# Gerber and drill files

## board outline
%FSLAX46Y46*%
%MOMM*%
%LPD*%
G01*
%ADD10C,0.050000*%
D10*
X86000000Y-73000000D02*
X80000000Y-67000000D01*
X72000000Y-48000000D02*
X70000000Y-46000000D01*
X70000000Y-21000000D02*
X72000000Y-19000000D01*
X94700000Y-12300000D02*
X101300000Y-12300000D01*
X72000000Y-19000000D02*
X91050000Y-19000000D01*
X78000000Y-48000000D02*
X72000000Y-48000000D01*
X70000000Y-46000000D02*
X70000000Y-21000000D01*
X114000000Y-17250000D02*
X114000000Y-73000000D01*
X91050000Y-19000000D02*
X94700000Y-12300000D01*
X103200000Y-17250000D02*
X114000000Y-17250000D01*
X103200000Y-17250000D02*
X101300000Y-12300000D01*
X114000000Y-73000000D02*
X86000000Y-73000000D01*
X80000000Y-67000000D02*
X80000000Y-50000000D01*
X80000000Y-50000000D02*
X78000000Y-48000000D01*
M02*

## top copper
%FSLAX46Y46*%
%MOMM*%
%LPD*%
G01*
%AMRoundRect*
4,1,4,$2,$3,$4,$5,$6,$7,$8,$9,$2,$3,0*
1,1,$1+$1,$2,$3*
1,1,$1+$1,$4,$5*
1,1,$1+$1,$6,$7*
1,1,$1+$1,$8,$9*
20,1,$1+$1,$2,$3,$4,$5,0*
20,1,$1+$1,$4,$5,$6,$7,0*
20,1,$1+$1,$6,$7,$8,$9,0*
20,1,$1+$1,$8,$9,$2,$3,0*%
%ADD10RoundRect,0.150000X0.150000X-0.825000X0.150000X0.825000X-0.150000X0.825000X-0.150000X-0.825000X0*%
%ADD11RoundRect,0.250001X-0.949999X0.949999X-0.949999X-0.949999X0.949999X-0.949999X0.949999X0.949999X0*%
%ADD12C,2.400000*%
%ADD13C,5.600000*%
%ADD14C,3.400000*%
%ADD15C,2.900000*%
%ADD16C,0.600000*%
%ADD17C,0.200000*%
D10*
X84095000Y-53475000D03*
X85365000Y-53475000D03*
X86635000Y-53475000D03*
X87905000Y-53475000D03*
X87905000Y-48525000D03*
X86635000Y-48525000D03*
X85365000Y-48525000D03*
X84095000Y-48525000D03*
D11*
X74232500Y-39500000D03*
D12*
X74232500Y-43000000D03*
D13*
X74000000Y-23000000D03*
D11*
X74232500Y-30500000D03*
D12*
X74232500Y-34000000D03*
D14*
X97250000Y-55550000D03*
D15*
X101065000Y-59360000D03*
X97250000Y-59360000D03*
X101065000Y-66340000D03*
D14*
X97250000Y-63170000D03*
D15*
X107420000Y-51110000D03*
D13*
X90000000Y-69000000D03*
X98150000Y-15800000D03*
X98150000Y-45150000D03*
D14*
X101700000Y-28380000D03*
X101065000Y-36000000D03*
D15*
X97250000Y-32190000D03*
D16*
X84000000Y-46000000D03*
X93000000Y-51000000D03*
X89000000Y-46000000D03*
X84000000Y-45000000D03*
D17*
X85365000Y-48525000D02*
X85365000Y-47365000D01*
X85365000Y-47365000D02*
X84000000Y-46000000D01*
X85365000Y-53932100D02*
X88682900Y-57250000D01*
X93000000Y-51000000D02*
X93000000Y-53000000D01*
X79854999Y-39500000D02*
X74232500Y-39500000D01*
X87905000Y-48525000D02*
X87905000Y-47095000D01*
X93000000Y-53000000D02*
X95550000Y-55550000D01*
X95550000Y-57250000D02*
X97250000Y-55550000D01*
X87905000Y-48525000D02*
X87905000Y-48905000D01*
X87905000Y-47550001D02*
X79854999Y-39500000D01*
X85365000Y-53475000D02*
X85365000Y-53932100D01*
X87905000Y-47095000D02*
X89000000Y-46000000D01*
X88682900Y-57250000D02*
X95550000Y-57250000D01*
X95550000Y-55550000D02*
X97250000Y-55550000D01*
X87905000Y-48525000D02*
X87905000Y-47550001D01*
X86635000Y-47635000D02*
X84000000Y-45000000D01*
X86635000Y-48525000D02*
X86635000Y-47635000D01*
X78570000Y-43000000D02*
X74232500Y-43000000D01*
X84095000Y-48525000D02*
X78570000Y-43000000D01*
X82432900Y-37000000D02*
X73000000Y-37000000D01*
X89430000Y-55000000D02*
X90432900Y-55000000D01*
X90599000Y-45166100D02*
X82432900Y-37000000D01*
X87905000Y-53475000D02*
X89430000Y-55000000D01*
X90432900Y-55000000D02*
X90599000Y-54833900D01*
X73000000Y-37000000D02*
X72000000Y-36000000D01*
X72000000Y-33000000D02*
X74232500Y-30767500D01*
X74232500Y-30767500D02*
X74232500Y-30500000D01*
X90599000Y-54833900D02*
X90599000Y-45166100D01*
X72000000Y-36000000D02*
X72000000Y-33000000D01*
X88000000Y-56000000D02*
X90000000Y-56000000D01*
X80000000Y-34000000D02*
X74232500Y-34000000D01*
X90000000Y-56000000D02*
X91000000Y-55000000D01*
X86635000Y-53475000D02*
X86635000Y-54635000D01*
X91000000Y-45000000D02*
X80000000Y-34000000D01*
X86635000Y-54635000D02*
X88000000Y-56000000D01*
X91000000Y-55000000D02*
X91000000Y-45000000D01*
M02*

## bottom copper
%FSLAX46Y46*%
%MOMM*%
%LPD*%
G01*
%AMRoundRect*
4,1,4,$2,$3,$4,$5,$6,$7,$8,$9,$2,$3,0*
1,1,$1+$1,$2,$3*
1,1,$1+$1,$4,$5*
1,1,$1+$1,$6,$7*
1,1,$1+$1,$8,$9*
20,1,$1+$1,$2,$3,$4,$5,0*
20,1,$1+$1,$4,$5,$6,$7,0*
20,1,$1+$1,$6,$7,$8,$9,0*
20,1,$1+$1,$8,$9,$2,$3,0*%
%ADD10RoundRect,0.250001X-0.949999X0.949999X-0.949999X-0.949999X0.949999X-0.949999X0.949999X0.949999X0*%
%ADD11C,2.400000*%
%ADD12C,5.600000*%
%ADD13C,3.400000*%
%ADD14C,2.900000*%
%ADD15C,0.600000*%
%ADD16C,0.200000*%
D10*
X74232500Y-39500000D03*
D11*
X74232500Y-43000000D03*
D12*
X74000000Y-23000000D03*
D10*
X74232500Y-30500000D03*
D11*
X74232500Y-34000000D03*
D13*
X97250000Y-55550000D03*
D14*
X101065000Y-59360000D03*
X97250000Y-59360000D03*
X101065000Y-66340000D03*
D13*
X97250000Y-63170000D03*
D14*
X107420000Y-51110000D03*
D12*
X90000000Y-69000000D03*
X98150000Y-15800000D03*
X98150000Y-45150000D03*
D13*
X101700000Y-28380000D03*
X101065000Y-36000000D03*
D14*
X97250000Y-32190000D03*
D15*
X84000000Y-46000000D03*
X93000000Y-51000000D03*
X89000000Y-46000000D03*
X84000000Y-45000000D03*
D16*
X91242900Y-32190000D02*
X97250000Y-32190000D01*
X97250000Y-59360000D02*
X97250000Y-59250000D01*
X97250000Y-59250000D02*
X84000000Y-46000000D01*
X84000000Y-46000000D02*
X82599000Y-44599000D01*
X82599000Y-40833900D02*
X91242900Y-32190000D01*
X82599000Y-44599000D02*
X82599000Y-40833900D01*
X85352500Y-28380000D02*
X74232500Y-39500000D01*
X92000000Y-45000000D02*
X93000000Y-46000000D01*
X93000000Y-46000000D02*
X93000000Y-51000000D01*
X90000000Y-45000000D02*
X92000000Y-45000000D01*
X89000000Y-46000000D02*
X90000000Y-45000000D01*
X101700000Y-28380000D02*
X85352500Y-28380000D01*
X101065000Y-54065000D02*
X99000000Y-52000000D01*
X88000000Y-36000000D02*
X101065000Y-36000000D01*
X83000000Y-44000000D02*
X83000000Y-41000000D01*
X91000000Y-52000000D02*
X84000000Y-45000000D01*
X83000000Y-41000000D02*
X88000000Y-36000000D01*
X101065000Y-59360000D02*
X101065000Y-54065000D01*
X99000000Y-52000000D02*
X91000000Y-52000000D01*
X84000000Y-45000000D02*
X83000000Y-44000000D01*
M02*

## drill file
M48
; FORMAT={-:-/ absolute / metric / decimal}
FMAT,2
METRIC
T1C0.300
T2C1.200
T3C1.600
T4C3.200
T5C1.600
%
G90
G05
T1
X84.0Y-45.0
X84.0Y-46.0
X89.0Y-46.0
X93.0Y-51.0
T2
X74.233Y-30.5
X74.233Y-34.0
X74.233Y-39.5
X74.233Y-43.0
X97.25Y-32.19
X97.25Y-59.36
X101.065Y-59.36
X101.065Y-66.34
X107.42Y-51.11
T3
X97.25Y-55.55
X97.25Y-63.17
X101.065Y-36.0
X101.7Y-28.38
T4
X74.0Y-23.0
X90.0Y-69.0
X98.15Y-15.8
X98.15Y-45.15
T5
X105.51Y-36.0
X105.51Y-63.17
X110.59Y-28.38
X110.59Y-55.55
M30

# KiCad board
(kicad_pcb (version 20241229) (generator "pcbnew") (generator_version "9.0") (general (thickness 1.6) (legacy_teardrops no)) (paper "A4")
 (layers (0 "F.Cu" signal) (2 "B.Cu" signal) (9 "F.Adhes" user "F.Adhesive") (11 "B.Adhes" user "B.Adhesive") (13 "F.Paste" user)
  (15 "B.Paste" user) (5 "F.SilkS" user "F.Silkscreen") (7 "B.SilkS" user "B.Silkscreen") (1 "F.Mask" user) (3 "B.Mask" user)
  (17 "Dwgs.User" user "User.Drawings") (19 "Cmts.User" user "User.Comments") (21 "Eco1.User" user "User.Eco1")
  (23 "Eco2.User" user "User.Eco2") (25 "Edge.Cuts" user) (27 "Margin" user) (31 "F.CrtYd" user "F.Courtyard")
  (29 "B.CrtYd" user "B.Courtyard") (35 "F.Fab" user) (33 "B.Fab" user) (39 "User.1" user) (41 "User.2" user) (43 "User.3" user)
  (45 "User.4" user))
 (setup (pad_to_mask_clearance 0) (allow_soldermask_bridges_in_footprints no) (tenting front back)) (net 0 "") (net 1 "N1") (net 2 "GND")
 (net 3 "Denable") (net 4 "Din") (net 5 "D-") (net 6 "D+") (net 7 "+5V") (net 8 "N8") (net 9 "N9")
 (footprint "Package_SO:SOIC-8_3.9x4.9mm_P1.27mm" (layer "F.Cu") (at 86 51 90)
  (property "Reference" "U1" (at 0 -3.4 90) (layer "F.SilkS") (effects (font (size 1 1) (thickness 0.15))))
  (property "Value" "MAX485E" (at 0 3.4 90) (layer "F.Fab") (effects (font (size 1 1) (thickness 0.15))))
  (pad "1" smd roundrect (at -2.475 -1.905 90) (size 1.95 0.6) (layers "F.Cu" "F.Mask" "F.Paste") (roundrect_rratio 0.25) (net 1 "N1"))
  (pad "2" smd roundrect (at -2.475 -0.635 90) (size 1.95 0.6) (layers "F.Cu" "F.Mask" "F.Paste") (roundrect_rratio 0.25) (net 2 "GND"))
  (pad "3" smd roundrect (at -2.475 0.635 90) (size 1.95 0.6) (layers "F.Cu" "F.Mask" "F.Paste") (roundrect_rratio 0.25) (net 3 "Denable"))
  (pad "4" smd roundrect (at -2.475 1.905 90) (size 1.95 0.6) (layers "F.Cu" "F.Mask" "F.Paste") (roundrect_rratio 0.25) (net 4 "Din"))
  (pad "5" smd roundrect (at 2.475 1.905 90) (size 1.95 0.6) (layers "F.Cu" "F.Mask" "F.Paste") (roundrect_rratio 0.25) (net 2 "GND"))
  (pad "6" smd roundrect (at 2.475 0.635 90) (size 1.95 0.6) (layers "F.Cu" "F.Mask" "F.Paste") (roundrect_rratio 0.25) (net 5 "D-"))
  (pad "7" smd roundrect (at 2.475 -0.635 90) (size 1.95 0.6) (layers "F.Cu" "F.Mask" "F.Paste") (roundrect_rratio 0.25) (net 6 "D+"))
  (pad "8" smd roundrect (at 2.475 -1.905 90) (size 1.95 0.6) (layers "F.Cu" "F.Mask" "F.Paste") (roundrect_rratio 0.25) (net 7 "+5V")))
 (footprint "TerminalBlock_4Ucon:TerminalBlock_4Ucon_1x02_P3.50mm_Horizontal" (layer "F.Cu") (at 74.2325 39.5 -90)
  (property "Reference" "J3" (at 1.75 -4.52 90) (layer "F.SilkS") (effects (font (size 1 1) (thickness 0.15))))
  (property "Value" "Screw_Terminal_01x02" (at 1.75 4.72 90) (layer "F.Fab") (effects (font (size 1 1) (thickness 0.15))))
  (pad "1" thru_hole roundrect (at 0 0 270) (size 2.4 2.4) (drill 1.2) (layers "*.Cu" "*.Mask") (remove_unused_layers no)
   (roundrect_rratio 0.104167) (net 2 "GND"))
  (pad "2" thru_hole circle (at 3.5 0 270) (size 2.4 2.4) (drill 1.2) (layers "*.Cu" "*.Mask") (remove_unused_layers no) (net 7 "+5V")))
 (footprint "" (layer "F.Cu") (at 74 23)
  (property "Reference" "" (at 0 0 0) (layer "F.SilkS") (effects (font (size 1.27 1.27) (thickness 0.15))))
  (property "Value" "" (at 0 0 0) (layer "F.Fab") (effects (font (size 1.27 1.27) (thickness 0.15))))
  (pad "1" thru_hole circle (at 0 0) (size 5.6 5.6) (drill 3.2) (layers "*.Cu" "*.Mask") (remove_unused_layers no) (zone_connect 2)))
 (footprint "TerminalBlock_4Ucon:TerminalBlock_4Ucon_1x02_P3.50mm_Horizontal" (layer "F.Cu") (at 74.2325 30.5 -90)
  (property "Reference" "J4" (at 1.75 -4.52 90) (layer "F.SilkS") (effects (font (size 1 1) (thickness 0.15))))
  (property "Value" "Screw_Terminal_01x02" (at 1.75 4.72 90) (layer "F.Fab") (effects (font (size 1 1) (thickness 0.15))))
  (pad "1" thru_hole roundrect (at 0 0 270) (size 2.4 2.4) (drill 1.2) (layers "*.Cu" "*.Mask") (remove_unused_layers no)
   (roundrect_rratio 0.104167) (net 4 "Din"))
  (pad "2" thru_hole circle (at 3.5 0 270) (size 2.4 2.4) (drill 1.2) (layers "*.Cu" "*.Mask") (remove_unused_layers no) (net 3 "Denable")))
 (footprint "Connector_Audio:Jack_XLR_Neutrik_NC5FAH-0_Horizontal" (layer "F.Cu") (at 97.25 55.55)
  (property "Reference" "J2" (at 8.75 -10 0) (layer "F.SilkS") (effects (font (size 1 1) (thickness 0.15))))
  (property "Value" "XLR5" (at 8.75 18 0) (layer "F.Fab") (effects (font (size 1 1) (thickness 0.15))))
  (pad "" np_thru_hole circle (at 8.26 7.62) (size 1.6 1.6) (drill 1.6) (layers "*.Cu" "*.Mask"))
  (pad "" np_thru_hole circle (at 13.34 0) (size 1.6 1.6) (drill 1.6) (layers "*.Cu" "*.Mask"))
  (pad "1" thru_hole circle (at 0 0) (size 3.4 3.4) (drill 1.6) (layers "*.Cu" "*.Mask") (remove_unused_layers no) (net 2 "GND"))
  (pad "2" thru_hole circle (at 3.815 3.81) (size 2.9 2.9) (drill 1.2) (layers "*.Cu" "*.Mask") (remove_unused_layers no) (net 5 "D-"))
  (pad "3" thru_hole circle (at 0 3.81) (size 2.9 2.9) (drill 1.2) (layers "*.Cu" "*.Mask") (remove_unused_layers no) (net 6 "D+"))
  (pad "4" thru_hole circle (at 3.815 10.79) (size 2.9 2.9) (drill 1.2) (layers "*.Cu" "*.Mask") (remove_unused_layers no) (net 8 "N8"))
  (pad "5" thru_hole circle (at 0 7.62) (size 3.4 3.4) (drill 1.6) (layers "*.Cu" "*.Mask") (remove_unused_layers no) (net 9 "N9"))
  (pad "G" thru_hole circle (at 10.17 -4.44) (size 2.9 2.9) (drill 1.2) (layers "*.Cu" "*.Mask") (remove_unused_layers no)))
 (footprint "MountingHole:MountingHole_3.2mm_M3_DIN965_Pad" (layer "F.Cu") (at 90 69)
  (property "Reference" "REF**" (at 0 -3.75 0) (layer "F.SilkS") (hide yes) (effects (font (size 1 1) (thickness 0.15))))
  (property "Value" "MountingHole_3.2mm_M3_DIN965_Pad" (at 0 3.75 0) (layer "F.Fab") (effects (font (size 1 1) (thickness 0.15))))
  (pad "1" thru_hole circle (at 0 0) (size 5.6 5.6) (drill 3.2) (layers "*.Cu" "*.Mask") (remove_unused_layers no) (zone_connect 2)))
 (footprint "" (layer "F.Cu") (at 98.15 15.8)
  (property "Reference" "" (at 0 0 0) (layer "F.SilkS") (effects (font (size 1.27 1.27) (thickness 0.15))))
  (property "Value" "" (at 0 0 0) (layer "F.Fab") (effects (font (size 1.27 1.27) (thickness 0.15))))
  (pad "1" thru_hole circle (at 0 0) (size 5.6 5.6) (drill 3.2) (layers "*.Cu" "*.Mask") (remove_unused_layers no) (zone_connect 2)))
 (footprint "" (layer "F.Cu") (at 98.15 45.15)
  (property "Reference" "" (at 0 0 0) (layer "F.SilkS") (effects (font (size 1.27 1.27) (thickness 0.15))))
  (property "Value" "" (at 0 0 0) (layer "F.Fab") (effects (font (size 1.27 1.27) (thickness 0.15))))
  (pad "1" thru_hole circle (at 0 0) (size 5.6 5.6) (drill 3.2) (layers "*.Cu" "*.Mask") (remove_unused_layers no) (zone_connect 2)))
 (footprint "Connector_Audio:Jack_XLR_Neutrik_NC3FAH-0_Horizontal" (layer "F.Cu") (at 101.7 28.38)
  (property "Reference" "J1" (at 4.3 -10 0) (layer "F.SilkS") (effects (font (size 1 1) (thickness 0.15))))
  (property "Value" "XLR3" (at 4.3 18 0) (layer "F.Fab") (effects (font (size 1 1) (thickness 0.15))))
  (pad "" np_thru_hole circle (at 3.81 7.62) (size 1.6 1.6) (drill 1.6) (layers "*.Cu" "*.Mask"))
  (pad "" np_thru_hole circle (at 8.89 0) (size 1.6 1.6) (drill 1.6) (layers "*.Cu" "*.Mask"))
  (pad "1" thru_hole circle (at 0 0) (size 3.4 3.4) (drill 1.6) (layers "*.Cu" "*.Mask") (remove_unused_layers no) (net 2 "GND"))
  (pad "2" thru_hole circle (at -0.635 7.62) (size 3.4 3.4) (drill 1.6) (layers "*.Cu" "*.Mask") (remove_unused_layers no) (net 5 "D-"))
  (pad "3" thru_hole circle (at -4.45 3.81) (size 2.9 2.9) (drill 1.2) (layers "*.Cu" "*.Mask") (remove_unused_layers no) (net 6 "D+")))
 (gr_line (start 86 73) (end 80 67) (stroke (width 0.05) (type default)) (layer "Edge.Cuts"))
 (gr_line (start 72 48) (end 70 46) (stroke (width 0.05) (type default)) (layer "Edge.Cuts"))
 (gr_line (start 70 21) (end 72 19) (stroke (width 0.05) (type default)) (layer "Edge.Cuts"))
 (gr_line (start 94.7 12.3) (end 101.3 12.3) (stroke (width 0.05) (type default)) (layer "Edge.Cuts"))
 (gr_line (start 72 19) (end 91.05 19) (stroke (width 0.05) (type default)) (layer "Edge.Cuts"))
 (gr_line (start 78 48) (end 72 48) (stroke (width 0.05) (type default)) (layer "Edge.Cuts"))
 (gr_line (start 70 46) (end 70 21) (stroke (width 0.05) (type default)) (layer "Edge.Cuts"))
 (gr_line (start 114 17.25) (end 114 73) (stroke (width 0.05) (type default)) (layer "Edge.Cuts"))
 (gr_line (start 91.05 19) (end 94.7 12.3) (stroke (width 0.05) (type default)) (layer "Edge.Cuts"))
 (gr_line (start 103.2 17.25) (end 114 17.25) (stroke (width 0.05) (type default)) (layer "Edge.Cuts"))
 (gr_line (start 103.2 17.25) (end 101.3 12.3) (stroke (width 0.05) (type default)) (layer "Edge.Cuts"))
 (gr_line (start 114 73) (end 86 73) (stroke (width 0.05) (type default)) (layer "Edge.Cuts"))
 (gr_line (start 80 67) (end 80 50) (stroke (width 0.05) (type default)) (layer "Edge.Cuts"))
 (gr_line (start 80 50) (end 78 48) (stroke (width 0.05) (type default)) (layer "Edge.Cuts"))
 (segment (start 85.365 48.525) (end 85.365 47.365) (width 0.2) (layer "F.Cu") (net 6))
 (segment (start 85.365 47.365) (end 84 46) (width 0.2) (layer "F.Cu") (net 6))
 (via (at 84 46) (size 0.6) (drill 0.3) (layers "F.Cu" "B.Cu") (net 6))
 (segment (start 91.2429 32.19) (end 97.25 32.19) (width 0.2) (layer "B.Cu") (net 6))
 (segment (start 97.25 59.36) (end 97.25 59.25) (width 0.2) (layer "B.Cu") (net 6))
 (segment (start 97.25 59.25) (end 84 46) (width 0.2) (layer "B.Cu") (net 6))
 (segment (start 84 46) (end 82.599 44.599) (width 0.2) (layer "B.Cu") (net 6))
 (segment (start 82.599 40.8339) (end 91.2429 32.19) (width 0.2) (layer "B.Cu") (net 6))
 (segment (start 82.599 44.599) (end 82.599 40.8339) (width 0.2) (layer "B.Cu") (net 6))
 (segment (start 85.365 53.9321) (end 88.6829 57.25) (width 0.2) (layer "F.Cu") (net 2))
 (segment (start 93 51) (end 93 53) (width 0.2) (layer "F.Cu") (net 2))
 (segment (start 79.854999 39.5) (end 74.2325 39.5) (width 0.2) (layer "F.Cu") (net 2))
 (segment (start 87.905 48.525) (end 87.905 47.095) (width 0.2) (layer "F.Cu") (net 2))
 (segment (start 93 53) (end 95.55 55.55) (width 0.2) (layer "F.Cu") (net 2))
 (segment (start 95.55 57.25) (end 97.25 55.55) (width 0.2) (layer "F.Cu") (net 2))
 (segment (start 87.905 48.525) (end 87.905 48.905) (width 0.2) (layer "F.Cu") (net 2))
 (segment (start 87.905 47.550001) (end 79.854999 39.5) (width 0.2) (layer "F.Cu") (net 2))
 (segment (start 85.365 53.475) (end 85.365 53.9321) (width 0.2) (layer "F.Cu") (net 2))
 (segment (start 87.905 47.095) (end 89 46) (width 0.2) (layer "F.Cu") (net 2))
 (segment (start 88.6829 57.25) (end 95.55 57.25) (width 0.2) (layer "F.Cu") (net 2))
 (segment (start 95.55 55.55) (end 97.25 55.55) (width 0.2) (layer "F.Cu") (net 2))
 (segment (start 87.905 48.525) (end 87.905 47.550001) (width 0.2) (layer "F.Cu") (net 2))
 (via (at 93 51) (size 0.6) (drill 0.3) (layers "F.Cu" "B.Cu") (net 2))
 (via (at 89 46) (size 0.6) (drill 0.3) (layers "F.Cu" "B.Cu") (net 2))
 (segment (start 85.3525 28.38) (end 74.2325 39.5) (width 0.2) (layer "B.Cu") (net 2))
 (segment (start 92 45) (end 93 46) (width 0.2) (layer "B.Cu") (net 2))
 (segment (start 93 46) (end 93 51) (width 0.2) (layer "B.Cu") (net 2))
 (segment (start 90 45) (end 92 45) (width 0.2) (layer "B.Cu") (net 2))
 (segment (start 89 46) (end 90 45) (width 0.2) (layer "B.Cu") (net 2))
 (segment (start 101.7 28.38) (end 85.3525 28.38) (width 0.2) (layer "B.Cu") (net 2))
 (segment (start 86.635 47.635) (end 84 45) (width 0.2) (layer "F.Cu") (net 5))
 (segment (start 86.635 48.525) (end 86.635 47.635) (width 0.2) (layer "F.Cu") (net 5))
 (via (at 84 45) (size 0.6) (drill 0.3) (layers "F.Cu" "B.Cu") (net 5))
 (segment (start 101.065 54.065) (end 99 52) (width 0.2) (layer "B.Cu") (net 5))
 (segment (start 88 36) (end 101.065 36) (width 0.2) (layer "B.Cu") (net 5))
 (segment (start 83 44) (end 83 41) (width 0.2) (layer "B.Cu") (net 5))
 (segment (start 91 52) (end 84 45) (width 0.2) (layer "B.Cu") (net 5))
 (segment (start 83 41) (end 88 36) (width 0.2) (layer "B.Cu") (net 5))
 (segment (start 101.065 59.36) (end 101.065 54.065) (width 0.2) (layer "B.Cu") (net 5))
 (segment (start 99 52) (end 91 52) (width 0.2) (layer "B.Cu") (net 5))
 (segment (start 84 45) (end 83 44) (width 0.2) (layer "B.Cu") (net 5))
 (segment (start 78.57 43) (end 74.2325 43) (width 0.2) (layer "F.Cu") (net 7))
 (segment (start 84.095 48.525) (end 78.57 43) (width 0.2) (layer "F.Cu") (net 7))
 (segment (start 82.4329 37) (end 73 37) (width 0.2) (layer "F.Cu") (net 4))
 (segment (start 89.43 55) (end 90.4329 55) (width 0.2) (layer "F.Cu") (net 4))
 (segment (start 90.599 45.1661) (end 82.4329 37) (width 0.2) (layer "F.Cu") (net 4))
 (segment (start 87.905 53.475) (end 89.43 55) (width 0.2) (layer "F.Cu") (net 4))
 (segment (start 90.4329 55) (end 90.599 54.8339) (width 0.2) (layer "F.Cu") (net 4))
 (segment (start 73 37) (end 72 36) (width 0.2) (layer "F.Cu") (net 4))
 (segment (start 72 33) (end 74.2325 30.7675) (width 0.2) (layer "F.Cu") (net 4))
 (segment (start 74.2325 30.7675) (end 74.2325 30.5) (width 0.2) (layer "F.Cu") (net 4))
 (segment (start 90.599 54.8339) (end 90.599 45.1661) (width 0.2) (layer "F.Cu") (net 4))
 (segment (start 72 36) (end 72 33) (width 0.2) (layer "F.Cu") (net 4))
 (segment (start 88 56) (end 90 56) (width 0.2) (layer "F.Cu") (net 3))
 (segment (start 80 34) (end 74.2325 34) (width 0.2) (layer "F.Cu") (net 3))
 (segment (start 90 56) (end 91 55) (width 0.2) (layer "F.Cu") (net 3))
 (segment (start 86.635 53.475) (end 86.635 54.635) (width 0.2) (layer "F.Cu") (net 3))
 (segment (start 91 45) (end 80 34) (width 0.2) (layer "F.Cu") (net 3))
 (segment (start 86.635 54.635) (end 88 56) (width 0.2) (layer "F.Cu") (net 3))
 (segment (start 91 55) (end 91 45) (width 0.2) (layer "F.Cu") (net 3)))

